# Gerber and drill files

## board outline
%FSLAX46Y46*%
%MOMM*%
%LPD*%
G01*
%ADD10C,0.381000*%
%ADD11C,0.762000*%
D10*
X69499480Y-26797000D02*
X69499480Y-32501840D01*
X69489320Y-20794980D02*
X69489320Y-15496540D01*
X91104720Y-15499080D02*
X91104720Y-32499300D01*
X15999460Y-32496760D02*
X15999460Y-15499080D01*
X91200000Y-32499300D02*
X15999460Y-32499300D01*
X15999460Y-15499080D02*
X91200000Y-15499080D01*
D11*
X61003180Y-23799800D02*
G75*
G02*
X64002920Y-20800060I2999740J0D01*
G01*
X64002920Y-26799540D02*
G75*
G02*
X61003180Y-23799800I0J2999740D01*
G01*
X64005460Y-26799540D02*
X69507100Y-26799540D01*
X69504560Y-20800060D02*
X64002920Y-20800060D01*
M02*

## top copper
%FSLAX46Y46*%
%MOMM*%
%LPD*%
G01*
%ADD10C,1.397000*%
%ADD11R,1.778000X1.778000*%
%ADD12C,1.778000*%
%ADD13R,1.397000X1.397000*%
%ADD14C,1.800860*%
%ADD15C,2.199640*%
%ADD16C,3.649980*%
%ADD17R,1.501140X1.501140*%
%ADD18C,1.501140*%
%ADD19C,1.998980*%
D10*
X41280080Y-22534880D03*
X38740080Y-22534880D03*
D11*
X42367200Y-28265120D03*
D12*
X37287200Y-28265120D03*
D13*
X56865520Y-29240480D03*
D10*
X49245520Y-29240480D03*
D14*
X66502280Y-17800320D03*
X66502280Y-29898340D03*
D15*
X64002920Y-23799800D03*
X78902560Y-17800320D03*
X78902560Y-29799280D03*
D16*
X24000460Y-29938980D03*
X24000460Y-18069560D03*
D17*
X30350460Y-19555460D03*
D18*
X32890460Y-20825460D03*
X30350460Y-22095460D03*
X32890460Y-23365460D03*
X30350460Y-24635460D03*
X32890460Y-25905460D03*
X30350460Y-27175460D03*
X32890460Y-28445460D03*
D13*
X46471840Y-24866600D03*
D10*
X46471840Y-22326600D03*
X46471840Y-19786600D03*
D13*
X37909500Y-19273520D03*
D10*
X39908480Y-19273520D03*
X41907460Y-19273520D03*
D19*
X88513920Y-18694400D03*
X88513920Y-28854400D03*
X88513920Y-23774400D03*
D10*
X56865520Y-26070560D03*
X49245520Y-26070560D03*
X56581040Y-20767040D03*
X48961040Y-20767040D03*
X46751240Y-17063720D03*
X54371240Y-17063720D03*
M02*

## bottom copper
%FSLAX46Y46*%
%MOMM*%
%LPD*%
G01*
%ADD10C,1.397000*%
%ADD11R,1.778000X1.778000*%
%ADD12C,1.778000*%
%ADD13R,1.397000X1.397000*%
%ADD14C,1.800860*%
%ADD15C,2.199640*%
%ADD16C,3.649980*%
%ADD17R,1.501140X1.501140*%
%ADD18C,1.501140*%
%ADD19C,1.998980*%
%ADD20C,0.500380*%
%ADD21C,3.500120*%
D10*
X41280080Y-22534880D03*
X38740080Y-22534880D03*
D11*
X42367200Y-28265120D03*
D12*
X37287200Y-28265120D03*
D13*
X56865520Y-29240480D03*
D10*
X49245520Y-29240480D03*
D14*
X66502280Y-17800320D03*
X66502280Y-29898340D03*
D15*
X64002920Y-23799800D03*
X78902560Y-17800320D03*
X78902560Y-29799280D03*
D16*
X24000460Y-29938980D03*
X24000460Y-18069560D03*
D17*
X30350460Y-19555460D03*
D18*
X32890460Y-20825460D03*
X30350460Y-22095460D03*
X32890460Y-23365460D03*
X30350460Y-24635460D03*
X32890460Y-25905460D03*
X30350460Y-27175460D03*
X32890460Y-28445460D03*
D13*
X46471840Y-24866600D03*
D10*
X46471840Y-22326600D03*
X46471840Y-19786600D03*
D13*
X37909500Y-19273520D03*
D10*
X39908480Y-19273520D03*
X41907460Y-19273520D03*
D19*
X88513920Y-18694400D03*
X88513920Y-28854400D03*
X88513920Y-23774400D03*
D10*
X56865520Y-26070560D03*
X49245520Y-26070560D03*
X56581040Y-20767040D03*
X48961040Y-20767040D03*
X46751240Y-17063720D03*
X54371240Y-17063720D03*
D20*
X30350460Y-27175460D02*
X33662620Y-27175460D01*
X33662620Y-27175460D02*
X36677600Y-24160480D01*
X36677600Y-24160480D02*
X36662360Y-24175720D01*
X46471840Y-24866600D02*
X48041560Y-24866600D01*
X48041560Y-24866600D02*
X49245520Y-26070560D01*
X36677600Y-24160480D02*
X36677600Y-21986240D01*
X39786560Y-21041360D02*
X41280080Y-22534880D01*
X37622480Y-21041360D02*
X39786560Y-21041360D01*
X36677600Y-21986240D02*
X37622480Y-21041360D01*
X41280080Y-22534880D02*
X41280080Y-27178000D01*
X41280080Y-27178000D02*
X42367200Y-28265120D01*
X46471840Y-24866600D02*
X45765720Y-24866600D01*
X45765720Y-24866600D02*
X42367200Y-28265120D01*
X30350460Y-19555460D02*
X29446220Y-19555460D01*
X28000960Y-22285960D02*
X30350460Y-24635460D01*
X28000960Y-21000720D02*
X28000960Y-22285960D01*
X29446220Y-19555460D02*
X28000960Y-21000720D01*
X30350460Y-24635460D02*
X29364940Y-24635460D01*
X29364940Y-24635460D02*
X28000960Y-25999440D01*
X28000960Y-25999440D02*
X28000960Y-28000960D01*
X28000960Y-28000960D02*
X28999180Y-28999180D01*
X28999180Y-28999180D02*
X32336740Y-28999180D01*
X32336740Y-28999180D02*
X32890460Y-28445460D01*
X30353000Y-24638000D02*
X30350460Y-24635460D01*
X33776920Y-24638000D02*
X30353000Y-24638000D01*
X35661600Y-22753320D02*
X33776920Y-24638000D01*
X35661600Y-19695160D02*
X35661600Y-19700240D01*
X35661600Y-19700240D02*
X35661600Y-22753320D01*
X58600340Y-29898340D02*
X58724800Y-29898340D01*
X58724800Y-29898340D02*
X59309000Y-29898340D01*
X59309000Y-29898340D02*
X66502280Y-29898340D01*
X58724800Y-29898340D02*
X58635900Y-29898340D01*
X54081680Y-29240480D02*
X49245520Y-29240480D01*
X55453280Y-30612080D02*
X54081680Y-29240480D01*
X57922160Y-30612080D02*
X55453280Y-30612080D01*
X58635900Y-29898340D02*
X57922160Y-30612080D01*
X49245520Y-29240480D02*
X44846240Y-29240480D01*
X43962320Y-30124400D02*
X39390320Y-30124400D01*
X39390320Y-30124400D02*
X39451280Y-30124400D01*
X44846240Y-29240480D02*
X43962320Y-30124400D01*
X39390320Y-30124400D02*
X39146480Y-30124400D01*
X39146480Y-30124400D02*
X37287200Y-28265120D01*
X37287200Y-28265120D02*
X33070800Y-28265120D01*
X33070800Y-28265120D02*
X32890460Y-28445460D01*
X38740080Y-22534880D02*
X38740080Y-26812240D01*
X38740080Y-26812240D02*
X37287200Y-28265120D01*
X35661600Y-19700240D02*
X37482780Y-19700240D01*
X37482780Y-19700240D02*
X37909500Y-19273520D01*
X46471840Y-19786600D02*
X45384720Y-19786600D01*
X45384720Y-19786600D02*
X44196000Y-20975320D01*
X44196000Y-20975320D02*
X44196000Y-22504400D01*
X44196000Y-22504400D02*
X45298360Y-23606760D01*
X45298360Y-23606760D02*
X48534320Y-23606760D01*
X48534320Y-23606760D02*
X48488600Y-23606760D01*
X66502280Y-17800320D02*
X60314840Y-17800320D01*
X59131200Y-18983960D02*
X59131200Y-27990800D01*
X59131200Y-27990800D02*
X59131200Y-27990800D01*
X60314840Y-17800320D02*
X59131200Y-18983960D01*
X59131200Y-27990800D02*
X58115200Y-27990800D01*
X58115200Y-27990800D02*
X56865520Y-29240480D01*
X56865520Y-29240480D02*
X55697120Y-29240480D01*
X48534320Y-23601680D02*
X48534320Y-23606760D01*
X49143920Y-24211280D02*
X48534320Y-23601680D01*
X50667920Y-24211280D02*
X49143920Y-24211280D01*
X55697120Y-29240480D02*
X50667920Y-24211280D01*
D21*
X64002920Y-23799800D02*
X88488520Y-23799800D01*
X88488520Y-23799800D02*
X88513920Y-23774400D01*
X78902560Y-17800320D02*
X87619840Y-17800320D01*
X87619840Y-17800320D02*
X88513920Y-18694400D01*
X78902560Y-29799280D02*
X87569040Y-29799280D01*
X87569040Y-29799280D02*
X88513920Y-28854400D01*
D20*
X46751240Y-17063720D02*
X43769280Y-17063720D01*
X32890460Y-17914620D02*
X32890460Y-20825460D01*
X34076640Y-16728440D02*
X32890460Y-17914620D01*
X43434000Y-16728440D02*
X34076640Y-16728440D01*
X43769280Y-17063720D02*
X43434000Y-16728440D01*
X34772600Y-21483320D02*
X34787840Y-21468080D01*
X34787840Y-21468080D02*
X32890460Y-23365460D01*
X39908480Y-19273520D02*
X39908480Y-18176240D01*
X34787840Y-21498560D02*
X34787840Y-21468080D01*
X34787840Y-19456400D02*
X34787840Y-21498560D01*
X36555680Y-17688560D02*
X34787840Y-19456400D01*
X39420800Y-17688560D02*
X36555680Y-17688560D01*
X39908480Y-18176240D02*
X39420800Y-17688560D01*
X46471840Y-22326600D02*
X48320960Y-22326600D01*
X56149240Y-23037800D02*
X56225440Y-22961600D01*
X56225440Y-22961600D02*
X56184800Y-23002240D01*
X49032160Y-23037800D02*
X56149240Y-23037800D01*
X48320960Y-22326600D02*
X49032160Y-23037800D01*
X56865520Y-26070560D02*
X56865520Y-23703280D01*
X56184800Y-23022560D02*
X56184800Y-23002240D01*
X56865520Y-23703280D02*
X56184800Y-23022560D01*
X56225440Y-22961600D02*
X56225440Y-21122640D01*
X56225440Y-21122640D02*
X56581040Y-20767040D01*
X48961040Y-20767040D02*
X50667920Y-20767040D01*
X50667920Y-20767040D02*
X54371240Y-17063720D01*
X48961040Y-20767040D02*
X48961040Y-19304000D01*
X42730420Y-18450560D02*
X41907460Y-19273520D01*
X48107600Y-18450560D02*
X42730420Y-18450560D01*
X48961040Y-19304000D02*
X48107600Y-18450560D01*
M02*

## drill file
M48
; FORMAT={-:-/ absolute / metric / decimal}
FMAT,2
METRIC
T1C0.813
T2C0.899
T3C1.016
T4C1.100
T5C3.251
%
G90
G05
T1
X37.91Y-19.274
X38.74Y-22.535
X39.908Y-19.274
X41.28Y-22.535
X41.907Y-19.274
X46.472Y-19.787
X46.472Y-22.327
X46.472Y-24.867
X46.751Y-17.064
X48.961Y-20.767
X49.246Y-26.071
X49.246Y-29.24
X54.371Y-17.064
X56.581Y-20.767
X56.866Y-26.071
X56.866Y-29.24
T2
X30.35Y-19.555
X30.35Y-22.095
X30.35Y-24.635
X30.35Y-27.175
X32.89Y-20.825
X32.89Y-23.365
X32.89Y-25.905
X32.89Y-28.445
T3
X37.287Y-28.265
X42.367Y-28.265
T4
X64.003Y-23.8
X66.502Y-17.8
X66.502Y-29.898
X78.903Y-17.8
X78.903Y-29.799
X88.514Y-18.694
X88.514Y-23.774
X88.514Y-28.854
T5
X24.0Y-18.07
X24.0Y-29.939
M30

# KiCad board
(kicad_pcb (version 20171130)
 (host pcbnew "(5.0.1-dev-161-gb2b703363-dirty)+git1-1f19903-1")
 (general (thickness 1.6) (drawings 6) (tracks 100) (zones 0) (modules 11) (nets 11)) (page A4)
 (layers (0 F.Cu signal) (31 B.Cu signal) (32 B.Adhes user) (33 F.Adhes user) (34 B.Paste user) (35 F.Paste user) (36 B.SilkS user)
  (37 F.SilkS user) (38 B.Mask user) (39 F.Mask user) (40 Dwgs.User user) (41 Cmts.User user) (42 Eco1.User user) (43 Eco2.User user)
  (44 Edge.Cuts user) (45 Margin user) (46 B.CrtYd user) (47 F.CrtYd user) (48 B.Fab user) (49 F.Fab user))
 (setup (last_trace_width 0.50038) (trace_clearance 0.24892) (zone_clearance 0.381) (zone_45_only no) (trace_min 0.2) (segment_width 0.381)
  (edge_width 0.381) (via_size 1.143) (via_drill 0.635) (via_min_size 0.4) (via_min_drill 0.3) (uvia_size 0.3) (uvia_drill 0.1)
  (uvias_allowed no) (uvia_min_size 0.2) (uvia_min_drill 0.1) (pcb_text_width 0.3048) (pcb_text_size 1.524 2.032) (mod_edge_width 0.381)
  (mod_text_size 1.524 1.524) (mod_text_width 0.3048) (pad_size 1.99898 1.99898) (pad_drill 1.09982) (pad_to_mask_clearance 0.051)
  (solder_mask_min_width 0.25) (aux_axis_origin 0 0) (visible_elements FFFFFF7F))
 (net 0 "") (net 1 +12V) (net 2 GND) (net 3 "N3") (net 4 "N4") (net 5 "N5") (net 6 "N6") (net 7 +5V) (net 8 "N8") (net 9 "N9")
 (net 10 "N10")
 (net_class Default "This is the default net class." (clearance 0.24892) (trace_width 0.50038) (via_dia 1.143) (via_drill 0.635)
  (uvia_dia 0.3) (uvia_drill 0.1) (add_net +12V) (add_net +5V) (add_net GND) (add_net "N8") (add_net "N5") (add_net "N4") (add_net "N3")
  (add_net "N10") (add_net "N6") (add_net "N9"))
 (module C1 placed (layer F.Cu) (at 40.01008 22.53488 180)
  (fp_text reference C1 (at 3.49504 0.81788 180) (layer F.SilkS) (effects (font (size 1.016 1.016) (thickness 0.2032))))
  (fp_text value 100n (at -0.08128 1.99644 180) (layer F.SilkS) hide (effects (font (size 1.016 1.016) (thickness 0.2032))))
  (pad 1 thru_hole circle (at -1.27 0 180) (size 1.397 1.397) (drill 0.8128) (layers *.Cu *.Mask F.SilkS) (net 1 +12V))
  (pad 2 thru_hole circle (at 1.27 0 180) (size 1.397 1.397) (drill 0.8128) (layers *.Cu *.Mask F.SilkS) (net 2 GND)))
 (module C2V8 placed (layer F.Cu) (at 39.8272 28.26512 180)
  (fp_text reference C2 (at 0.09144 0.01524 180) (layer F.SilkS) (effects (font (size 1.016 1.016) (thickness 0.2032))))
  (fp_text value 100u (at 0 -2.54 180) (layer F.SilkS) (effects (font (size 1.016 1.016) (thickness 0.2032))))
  (pad 1 thru_hole rect (at -2.54 0 180) (size 1.778 1.778) (drill 1.016) (layers *.Cu *.Mask F.SilkS) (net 1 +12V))
  (pad 2 thru_hole circle (at 2.54 0 180) (size 1.778 1.778) (drill 1.016) (layers *.Cu *.Mask F.SilkS) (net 2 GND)))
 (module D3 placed (layer F.Cu) (at 53.05552 29.24048)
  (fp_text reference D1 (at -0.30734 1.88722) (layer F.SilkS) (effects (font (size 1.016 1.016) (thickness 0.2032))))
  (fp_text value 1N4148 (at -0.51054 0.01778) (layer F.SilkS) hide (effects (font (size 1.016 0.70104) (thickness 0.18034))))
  (pad 2 thru_hole rect (at 3.81 0) (size 1.397 1.397) (drill 0.8128) (layers *.Cu *.Mask F.SilkS) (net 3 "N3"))
  (pad 1 thru_hole circle (at -3.81 0) (size 1.397 1.397) (drill 0.8128) (layers *.Cu *.Mask F.SilkS) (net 2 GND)))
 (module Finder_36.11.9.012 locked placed (layer F.Cu) (at 62.60338 15.99946 270) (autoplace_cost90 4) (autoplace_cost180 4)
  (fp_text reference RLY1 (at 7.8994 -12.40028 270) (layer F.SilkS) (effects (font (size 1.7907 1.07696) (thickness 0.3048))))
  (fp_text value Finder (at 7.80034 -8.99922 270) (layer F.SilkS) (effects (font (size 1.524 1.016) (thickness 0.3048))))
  (fp_arc (start 7.80034 -1.39954) (end 7.80034 1.6002) (angle 90) (layer Edge.Cuts) (width 0.762))
  (fp_arc (start 7.80034 -1.39954) (end 10.80008 -1.39954) (angle 90) (layer Edge.Cuts) (width 0.762))
  (fp_line (start 10.80008 -1.40208) (end 10.80008 -6.90372) (layer Edge.Cuts) (width 0.762))
  (fp_line (start 4.8006 -6.90118) (end 4.8006 -1.39954) (layer Edge.Cuts) (width 0.762))
  (pad 1 thru_hole circle (at 1.80086 -3.8989 270) (size 1.80086 1.80086) (drill 1.09982) (layers *.Cu *.Mask F.SilkS) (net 3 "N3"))
  (pad 2 thru_hole circle (at 13.89888 -3.8989 270) (size 1.80086 1.80086) (drill 1.09982) (layers *.Cu *.Mask F.SilkS) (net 2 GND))
  (pad 3 thru_hole circle (at 7.80034 -1.39954 270) (size 2.19964 2.19964) (drill 1.09982) (layers *.Cu *.Mask F.SilkS) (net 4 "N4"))
  (pad 4 thru_hole circle (at 1.80086 -16.29918 270) (size 2.19964 2.19964) (drill 1.09982) (layers *.Cu *.Mask F.SilkS) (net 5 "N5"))
  (pad 5 thru_hole circle (at 13.79982 -16.29918 270) (size 2.19964 2.19964) (drill 1.09982) (layers *.Cu *.Mask F.SilkS) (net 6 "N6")))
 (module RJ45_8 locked (layer F.Cu) (at 24.00046 24.00046 270)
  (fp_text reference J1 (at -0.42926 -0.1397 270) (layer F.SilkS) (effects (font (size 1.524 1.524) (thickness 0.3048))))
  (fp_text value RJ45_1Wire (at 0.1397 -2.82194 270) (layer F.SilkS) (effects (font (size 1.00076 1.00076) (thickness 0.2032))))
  (pad Hole np_thru_hole circle (at 5.93852 0 270) (size 3.64998 3.64998) (drill 3.2512) (layers *.Cu *.SilkS *.Mask))
  (pad Hole np_thru_hole circle (at -5.9309 0 270) (size 3.64998 3.64998) (drill 3.2512) (layers *.Cu *.SilkS *.Mask))
  (pad 1 thru_hole rect (at -4.445 -6.35 270) (size 1.50114 1.50114) (drill 0.89916) (layers *.Cu *.Mask F.SilkS) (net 2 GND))
  (pad 2 thru_hole circle (at -3.175 -8.89 270) (size 1.50114 1.50114) (drill 0.89916) (layers *.Cu *.Mask F.SilkS) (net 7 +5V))
  (pad 3 thru_hole circle (at -1.905 -6.35 270) (size 1.50114 1.50114) (drill 0.89916) (layers *.Cu *.Mask F.SilkS))
  (pad 4 thru_hole circle (at -0.635 -8.89 270) (size 1.50114 1.50114) (drill 0.89916) (layers *.Cu *.Mask F.SilkS) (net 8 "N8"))
  (pad 5 thru_hole circle (at 0.635 -6.35 270) (size 1.50114 1.50114) (drill 0.89916) (layers *.Cu *.Mask F.SilkS) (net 2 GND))
  (pad 6 thru_hole circle (at 1.905 -8.89 270) (size 1.50114 1.50114) (drill 0.89916) (layers *.Cu *.Mask F.SilkS))
  (pad 7 thru_hole circle (at 3.175 -6.35 270) (size 1.50114 1.50114) (drill 0.89916) (layers *.Cu *.Mask F.SilkS) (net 1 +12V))
  (pad 8 thru_hole circle (at 4.445 -8.89 270) (size 1.50114 1.50114) (drill 0.89916) (layers *.Cu *.Mask F.SilkS) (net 2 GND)))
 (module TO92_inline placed (layer F.Cu) (at 46.47184 22.3266 90)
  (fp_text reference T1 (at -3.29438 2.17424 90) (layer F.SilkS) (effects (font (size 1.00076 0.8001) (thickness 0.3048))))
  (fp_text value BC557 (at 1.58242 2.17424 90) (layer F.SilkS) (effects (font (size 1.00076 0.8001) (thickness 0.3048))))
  (pad 1 thru_hole rect (at -2.54 0 90) (size 1.397 1.397) (drill 0.8128) (layers *.Cu *.Mask F.SilkS) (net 1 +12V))
  (pad 2 thru_hole circle (at 0 0 90) (size 1.397 1.397) (drill 0.8128) (layers *.Cu *.Mask F.SilkS) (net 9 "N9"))
  (pad 3 thru_hole circle (at 2.54 0 90) (size 1.397 1.397) (drill 0.8128) (layers *.Cu *.Mask F.SilkS) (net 3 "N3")))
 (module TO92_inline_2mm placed (layer F.Cu) (at 39.90848 19.27352)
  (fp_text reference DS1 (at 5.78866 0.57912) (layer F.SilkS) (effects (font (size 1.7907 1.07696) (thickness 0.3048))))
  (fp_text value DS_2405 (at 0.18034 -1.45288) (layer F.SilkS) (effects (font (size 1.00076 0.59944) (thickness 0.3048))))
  (pad 1 thru_hole rect (at -1.99898 0) (size 1.397 1.397) (drill 0.8128) (layers *.Cu *.Mask F.SilkS) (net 2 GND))
  (pad 2 thru_hole circle (at 0 0) (size 1.397 1.397) (drill 0.8128) (layers *.Cu *.Mask F.SilkS) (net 8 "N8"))
  (pad 3 thru_hole circle (at 1.99898 0) (size 1.397 1.397) (drill 0.8128) (layers *.Cu *.Mask F.SilkS) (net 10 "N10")))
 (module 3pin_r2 (layer F.Cu) (at 88.51392 23.7744 270)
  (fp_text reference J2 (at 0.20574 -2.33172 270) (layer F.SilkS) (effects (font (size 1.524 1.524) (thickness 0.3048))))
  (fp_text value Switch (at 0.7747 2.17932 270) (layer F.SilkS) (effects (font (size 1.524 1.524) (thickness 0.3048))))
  (pad 1 thru_hole circle (at -5.08 0 270) (size 1.99898 1.99898) (drill 1.09982) (layers *.Cu *.Mask F.SilkS) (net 5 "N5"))
  (pad 3 thru_hole circle (at 5.08 0 270) (size 1.99898 1.99898) (drill 1.09982) (layers *.Cu *.Mask F.SilkS) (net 6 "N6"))
  (pad 2 thru_hole circle (at 0 0 270) (size 1.99898 1.99898) (drill 1.09982) (layers *.Cu *.Mask F.SilkS) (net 4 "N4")))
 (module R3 (layer F.Cu) (at 53.05552 26.07056 180) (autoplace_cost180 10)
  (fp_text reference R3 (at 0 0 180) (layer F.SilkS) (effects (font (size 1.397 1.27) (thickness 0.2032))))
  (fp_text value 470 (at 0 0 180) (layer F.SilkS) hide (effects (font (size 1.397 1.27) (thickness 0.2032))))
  (pad 1 thru_hole circle (at -3.81 0 180) (size 1.397 1.397) (drill 0.8128) (layers *.Cu *.Mask F.SilkS) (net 9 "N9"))
  (pad 2 thru_hole circle (at 3.81 0 180) (size 1.397 1.397) (drill 0.8128) (layers *.Cu *.Mask F.SilkS) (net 1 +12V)))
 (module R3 (layer F.Cu) (at 52.77104 20.76704 180) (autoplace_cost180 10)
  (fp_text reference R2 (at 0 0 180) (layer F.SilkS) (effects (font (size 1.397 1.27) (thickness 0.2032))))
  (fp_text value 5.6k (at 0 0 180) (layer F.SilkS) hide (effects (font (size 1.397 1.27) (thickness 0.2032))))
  (pad 1 thru_hole circle (at -3.81 0 180) (size 1.397 1.397) (drill 0.8128) (layers *.Cu *.Mask F.SilkS) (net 9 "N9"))
  (pad 2 thru_hole circle (at 3.81 0 180) (size 1.397 1.397) (drill 0.8128) (layers *.Cu *.Mask F.SilkS) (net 10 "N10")))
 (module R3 (layer F.Cu) (at 50.56124 17.06372) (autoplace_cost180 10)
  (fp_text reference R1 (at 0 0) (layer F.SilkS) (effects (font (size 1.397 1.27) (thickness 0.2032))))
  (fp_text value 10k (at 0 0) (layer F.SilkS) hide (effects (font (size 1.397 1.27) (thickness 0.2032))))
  (pad 1 thru_hole circle (at -3.81 0) (size 1.397 1.397) (drill 0.8128) (layers *.Cu *.Mask F.SilkS) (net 7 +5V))
  (pad 2 thru_hole circle (at 3.81 0) (size 1.397 1.397) (drill 0.8128) (layers *.Cu *.Mask F.SilkS) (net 10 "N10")))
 (gr_line (start 69.49948 26.797) (end 69.49948 32.50184) (angle 90) (layer Edge.Cuts) (width 0.381))
 (gr_line (start 69.48932 20.79498) (end 69.48932 15.49654) (angle 90) (layer Edge.Cuts) (width 0.381))
 (gr_line (start 91.10472 15.49908) (end 91.10472 32.4993) (angle 90) (layer Edge.Cuts) (width 0.381))
 (gr_line (start 15.99946 32.49676) (end 15.99946 15.49908) (angle 90) (layer Edge.Cuts) (width 0.381))
 (gr_line (start 91.2 32.4993) (end 15.99946 32.4993) (angle 90) (layer Edge.Cuts) (width 0.381))
 (gr_line (start 15.99946 15.49908) (end 91.2 15.49908) (angle 90) (layer Edge.Cuts) (width 0.381))
 (segment (start 30.35046 27.17546) (end 33.66262 27.17546) (width 0.50038) (layer B.Cu) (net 1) (status 800))
 (segment (start 33.66262 27.17546) (end 36.6776 24.16048) (width 0.50038) (layer B.Cu) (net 1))
 (segment (start 36.6776 24.16048) (end 36.66236 24.17572) (width 0.50038) (layer B.Cu) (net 1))
 (segment (start 46.47184 24.8666) (end 48.04156 24.8666) (width 0.50038) (layer B.Cu) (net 1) (status 800))
 (segment (start 48.04156 24.8666) (end 49.24552 26.07056) (width 0.50038) (layer B.Cu) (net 1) (status 400))
 (segment (start 36.6776 24.16048) (end 36.6776 21.98624) (width 0.50038) (layer B.Cu) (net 1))
 (segment (start 39.78656 21.04136) (end 41.28008 22.53488) (width 0.50038) (layer B.Cu) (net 1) (status 400))
 (segment (start 37.62248 21.04136) (end 39.78656 21.04136) (width 0.50038) (layer B.Cu) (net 1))
 (segment (start 36.6776 21.98624) (end 37.62248 21.04136) (width 0.50038) (layer B.Cu) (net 1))
 (segment (start 41.28008 22.53488) (end 41.28008 27.178) (width 0.50038) (layer B.Cu) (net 1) (status 800))
 (segment (start 41.28008 27.178) (end 42.3672 28.26512) (width 0.50038) (layer B.Cu) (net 1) (status 400))
 (segment (start 46.47184 24.8666) (end 45.76572 24.8666) (width 0.50038) (layer B.Cu) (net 1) (status 800))
 (segment (start 45.76572 24.8666) (end 42.3672 28.26512) (width 0.50038) (layer B.Cu) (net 1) (status 400))
 (segment (start 30.35046 19.55546) (end 29.44622 19.55546) (width 0.50038) (layer B.Cu) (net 2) (status 800))
 (segment (start 28.00096 22.28596) (end 30.35046 24.63546) (width 0.50038) (layer B.Cu) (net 2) (status 400))
 (segment (start 28.00096 21.00072) (end 28.00096 22.28596) (width 0.50038) (layer B.Cu) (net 2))
 (segment (start 29.44622 19.55546) (end 28.00096 21.00072) (width 0.50038) (layer B.Cu) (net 2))
 (segment (start 30.35046 24.63546) (end 29.36494 24.63546) (width 0.50038) (layer B.Cu) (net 2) (status 800))
 (segment (start 29.36494 24.63546) (end 28.00096 25.99944) (width 0.50038) (layer B.Cu) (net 2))
 (segment (start 28.00096 25.99944) (end 28.00096 28.00096) (width 0.50038) (layer B.Cu) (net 2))
 (segment (start 28.00096 28.00096) (end 28.99918 28.99918) (width 0.50038) (layer B.Cu) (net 2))
 (segment (start 28.99918 28.99918) (end 32.33674 28.99918) (width 0.50038) (layer B.Cu) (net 2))
 (segment (start 32.33674 28.99918) (end 32.89046 28.44546) (width 0.50038) (layer B.Cu) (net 2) (status 400))
 (segment (start 30.353 24.638) (end 30.35046 24.63546) (width 0.50038) (layer B.Cu) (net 2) (status 400))
 (segment (start 33.77692 24.638) (end 30.353 24.638) (width 0.50038) (layer B.Cu) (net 2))
 (segment (start 35.6616 22.75332) (end 33.77692 24.638) (width 0.50038) (layer B.Cu) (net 2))
 (segment (start 35.6616 19.69516) (end 35.6616 19.70024) (width 0.50038) (layer B.Cu) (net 2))
 (segment (start 35.6616 19.70024) (end 35.6616 22.75332) (width 0.50038) (layer B.Cu) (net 2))
 (segment (start 58.60034 29.89834) (end 58.7248 29.89834) (width 0.50038) (layer B.Cu) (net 2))
 (segment (start 58.7248 29.89834) (end 59.309 29.89834) (width 0.50038) (layer B.Cu) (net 2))
 (segment (start 59.309 29.89834) (end 66.50228 29.89834) (width 0.50038) (layer B.Cu) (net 2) (status 400))
 (segment (start 58.7248 29.89834) (end 58.6359 29.89834) (width 0.50038) (layer B.Cu) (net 2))
 (segment (start 54.08168 29.24048) (end 49.24552 29.24048) (width 0.50038) (layer B.Cu) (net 2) (status 400))
 (segment (start 55.45328 30.61208) (end 54.08168 29.24048) (width 0.50038) (layer B.Cu) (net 2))
 (segment (start 57.92216 30.61208) (end 55.45328 30.61208) (width 0.50038) (layer B.Cu) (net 2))
 (segment (start 58.6359 29.89834) (end 57.92216 30.61208) (width 0.50038) (layer B.Cu) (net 2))
 (segment (start 49.24552 29.24048) (end 44.84624 29.24048) (width 0.50038) (layer B.Cu) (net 2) (status 800))
 (segment (start 43.96232 30.1244) (end 39.39032 30.1244) (width 0.50038) (layer B.Cu) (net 2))
 (segment (start 39.39032 30.1244) (end 39.45128 30.1244) (width 0.50038) (layer B.Cu) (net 2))
 (segment (start 44.84624 29.24048) (end 43.96232 30.1244) (width 0.50038) (layer B.Cu) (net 2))
 (segment (start 39.39032 30.1244) (end 39.14648 30.1244) (width 0.50038) (layer B.Cu) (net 2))
 (segment (start 39.14648 30.1244) (end 37.2872 28.26512) (width 0.50038) (layer B.Cu) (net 2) (status 400))
 (segment (start 37.2872 28.26512) (end 33.0708 28.26512) (width 0.50038) (layer B.Cu) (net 2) (status 800))
 (segment (start 33.0708 28.26512) (end 32.89046 28.44546) (width 0.50038) (layer B.Cu) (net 2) (status 400))
 (segment (start 38.74008 22.53488) (end 38.74008 26.81224) (width 0.50038) (layer B.Cu) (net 2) (status 800))
 (segment (start 38.74008 26.81224) (end 37.2872 28.26512) (width 0.50038) (layer B.Cu) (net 2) (status 400))
 (segment (start 35.6616 19.70024) (end 37.48278 19.70024) (width 0.50038) (layer B.Cu) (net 2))
 (segment (start 37.48278 19.70024) (end 37.9095 19.27352) (width 0.50038) (layer B.Cu) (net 2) (status 400))
 (segment (start 46.47184 19.7866) (end 45.38472 19.7866) (width 0.50038) (layer B.Cu) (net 3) (status 800))
 (segment (start 45.38472 19.7866) (end 44.196 20.97532) (width 0.50038) (layer B.Cu) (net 3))
 (segment (start 44.196 20.97532) (end 44.196 22.5044) (width 0.50038) (layer B.Cu) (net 3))
 (segment (start 44.196 22.5044) (end 45.29836 23.60676) (width 0.50038) (layer B.Cu) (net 3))
 (segment (start 45.29836 23.60676) (end 48.53432 23.60676) (width 0.50038) (layer B.Cu) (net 3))
 (segment (start 48.53432 23.60676) (end 48.4886 23.60676) (width 0.50038) (layer B.Cu) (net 3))
 (segment (start 66.50228 17.80032) (end 60.31484 17.80032) (width 0.50038) (layer B.Cu) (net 3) (status 800))
 (segment (start 59.1312 18.98396) (end 59.1312 27.9908) (width 0.50038) (layer B.Cu) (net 3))
 (segment (start 59.1312 27.9908) (end 59.1312 27.9908) (width 0.50038) (layer B.Cu) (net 3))
 (segment (start 60.31484 17.80032) (end 59.1312 18.98396) (width 0.50038) (layer B.Cu) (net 3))
 (segment (start 59.1312 27.9908) (end 58.1152 27.9908) (width 0.50038) (layer B.Cu) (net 3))
 (segment (start 58.1152 27.9908) (end 56.86552 29.24048) (width 0.50038) (layer B.Cu) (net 3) (status 400))
 (segment (start 56.86552 29.24048) (end 55.69712 29.24048) (width 0.50038) (layer B.Cu) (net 3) (status 800))
 (segment (start 48.53432 23.60168) (end 48.53432 23.60676) (width 0.50038) (layer B.Cu) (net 3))
 (segment (start 49.14392 24.21128) (end 48.53432 23.60168) (width 0.50038) (layer B.Cu) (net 3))
 (segment (start 50.66792 24.21128) (end 49.14392 24.21128) (width 0.50038) (layer B.Cu) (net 3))
 (segment (start 55.69712 29.24048) (end 50.66792 24.21128) (width 0.50038) (layer B.Cu) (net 3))
 (segment (start 64.00292 23.7998) (end 88.48852 23.7998) (width 3.50012) (layer B.Cu) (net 4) (status 800))
 (segment (start 88.48852 23.7998) (end 88.51392 23.7744) (width 3.50012) (layer B.Cu) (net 4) (status 400))
 (segment (start 78.90256 17.80032) (end 87.61984 17.80032) (width 3.50012) (layer B.Cu) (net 5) (status 800))
 (segment (start 87.61984 17.80032) (end 88.51392 18.6944) (width 3.50012) (layer B.Cu) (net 5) (status 400))
 (segment (start 78.90256 29.79928) (end 87.56904 29.79928) (width 3.50012) (layer B.Cu) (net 6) (status 800))
 (segment (start 87.56904 29.79928) (end 88.51392 28.8544) (width 3.50012) (layer B.Cu) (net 6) (status 400))
 (segment (start 46.75124 17.06372) (end 43.76928 17.06372) (width 0.50038) (layer B.Cu) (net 7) (status 800))
 (segment (start 32.89046 17.91462) (end 32.89046 20.82546) (width 0.50038) (layer B.Cu) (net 7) (status 400))
 (segment (start 34.07664 16.72844) (end 32.89046 17.91462) (width 0.50038) (layer B.Cu) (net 7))
 (segment (start 43.434 16.72844) (end 34.07664 16.72844) (width 0.50038) (layer B.Cu) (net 7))
 (segment (start 43.76928 17.06372) (end 43.434 16.72844) (width 0.50038) (layer B.Cu) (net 7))
 (segment (start 34.7726 21.48332) (end 34.78784 21.46808) (width 0.50038) (layer B.Cu) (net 8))
 (segment (start 34.78784 21.46808) (end 32.89046 23.36546) (width 0.50038) (layer B.Cu) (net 8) (status 400))
 (segment (start 39.90848 19.27352) (end 39.90848 18.17624) (width 0.50038) (layer B.Cu) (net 8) (status 800))
 (segment (start 34.78784 21.49856) (end 34.78784 21.46808) (width 0.50038) (layer B.Cu) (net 8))
 (segment (start 34.78784 19.4564) (end 34.78784 21.49856) (width 0.50038) (layer B.Cu) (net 8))
 (segment (start 36.55568 17.68856) (end 34.78784 19.4564) (width 0.50038) (layer B.Cu) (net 8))
 (segment (start 39.4208 17.68856) (end 36.55568 17.68856) (width 0.50038) (layer B.Cu) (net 8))
 (segment (start 39.90848 18.17624) (end 39.4208 17.68856) (width 0.50038) (layer B.Cu) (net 8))
 (segment (start 46.47184 22.3266) (end 48.32096 22.3266) (width 0.50038) (layer B.Cu) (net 9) (status 800))
 (segment (start 56.14924 23.0378) (end 56.22544 22.9616) (width 0.50038) (layer B.Cu) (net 9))
 (segment (start 56.22544 22.9616) (end 56.1848 23.00224) (width 0.50038) (layer B.Cu) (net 9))
 (segment (start 49.03216 23.0378) (end 56.14924 23.0378) (width 0.50038) (layer B.Cu) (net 9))
 (segment (start 48.32096 22.3266) (end 49.03216 23.0378) (width 0.50038) (layer B.Cu) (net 9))
 (segment (start 56.86552 26.07056) (end 56.86552 23.70328) (width 0.50038) (layer B.Cu) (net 9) (status 800))
 (segment (start 56.1848 23.02256) (end 56.1848 23.00224) (width 0.50038) (layer B.Cu) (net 9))
 (segment (start 56.86552 23.70328) (end 56.1848 23.02256) (width 0.50038) (layer B.Cu) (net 9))
 (segment (start 56.22544 22.9616) (end 56.22544 21.12264) (width 0.50038) (layer B.Cu) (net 9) (status 400))
 (segment (start 56.22544 21.12264) (end 56.58104 20.76704) (width 0.50038) (layer B.Cu) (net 9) (status C00))
 (segment (start 48.96104 20.76704) (end 50.66792 20.76704) (width 0.50038) (layer B.Cu) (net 10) (status 800))
 (segment (start 50.66792 20.76704) (end 54.37124 17.06372) (width 0.50038) (layer B.Cu) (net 10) (status 400))
 (segment (start 48.96104 20.76704) (end 48.96104 19.304) (width 0.50038) (layer B.Cu) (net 10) (status 800))
 (segment (start 42.73042 18.45056) (end 41.90746 19.27352) (width 0.50038) (layer B.Cu) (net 10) (status 400))
 (segment (start 48.1076 18.45056) (end 42.73042 18.45056) (width 0.50038) (layer B.Cu) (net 10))
 (segment (start 48.96104 19.304) (end 48.1076 18.45056) (width 0.50038) (layer B.Cu) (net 10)))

